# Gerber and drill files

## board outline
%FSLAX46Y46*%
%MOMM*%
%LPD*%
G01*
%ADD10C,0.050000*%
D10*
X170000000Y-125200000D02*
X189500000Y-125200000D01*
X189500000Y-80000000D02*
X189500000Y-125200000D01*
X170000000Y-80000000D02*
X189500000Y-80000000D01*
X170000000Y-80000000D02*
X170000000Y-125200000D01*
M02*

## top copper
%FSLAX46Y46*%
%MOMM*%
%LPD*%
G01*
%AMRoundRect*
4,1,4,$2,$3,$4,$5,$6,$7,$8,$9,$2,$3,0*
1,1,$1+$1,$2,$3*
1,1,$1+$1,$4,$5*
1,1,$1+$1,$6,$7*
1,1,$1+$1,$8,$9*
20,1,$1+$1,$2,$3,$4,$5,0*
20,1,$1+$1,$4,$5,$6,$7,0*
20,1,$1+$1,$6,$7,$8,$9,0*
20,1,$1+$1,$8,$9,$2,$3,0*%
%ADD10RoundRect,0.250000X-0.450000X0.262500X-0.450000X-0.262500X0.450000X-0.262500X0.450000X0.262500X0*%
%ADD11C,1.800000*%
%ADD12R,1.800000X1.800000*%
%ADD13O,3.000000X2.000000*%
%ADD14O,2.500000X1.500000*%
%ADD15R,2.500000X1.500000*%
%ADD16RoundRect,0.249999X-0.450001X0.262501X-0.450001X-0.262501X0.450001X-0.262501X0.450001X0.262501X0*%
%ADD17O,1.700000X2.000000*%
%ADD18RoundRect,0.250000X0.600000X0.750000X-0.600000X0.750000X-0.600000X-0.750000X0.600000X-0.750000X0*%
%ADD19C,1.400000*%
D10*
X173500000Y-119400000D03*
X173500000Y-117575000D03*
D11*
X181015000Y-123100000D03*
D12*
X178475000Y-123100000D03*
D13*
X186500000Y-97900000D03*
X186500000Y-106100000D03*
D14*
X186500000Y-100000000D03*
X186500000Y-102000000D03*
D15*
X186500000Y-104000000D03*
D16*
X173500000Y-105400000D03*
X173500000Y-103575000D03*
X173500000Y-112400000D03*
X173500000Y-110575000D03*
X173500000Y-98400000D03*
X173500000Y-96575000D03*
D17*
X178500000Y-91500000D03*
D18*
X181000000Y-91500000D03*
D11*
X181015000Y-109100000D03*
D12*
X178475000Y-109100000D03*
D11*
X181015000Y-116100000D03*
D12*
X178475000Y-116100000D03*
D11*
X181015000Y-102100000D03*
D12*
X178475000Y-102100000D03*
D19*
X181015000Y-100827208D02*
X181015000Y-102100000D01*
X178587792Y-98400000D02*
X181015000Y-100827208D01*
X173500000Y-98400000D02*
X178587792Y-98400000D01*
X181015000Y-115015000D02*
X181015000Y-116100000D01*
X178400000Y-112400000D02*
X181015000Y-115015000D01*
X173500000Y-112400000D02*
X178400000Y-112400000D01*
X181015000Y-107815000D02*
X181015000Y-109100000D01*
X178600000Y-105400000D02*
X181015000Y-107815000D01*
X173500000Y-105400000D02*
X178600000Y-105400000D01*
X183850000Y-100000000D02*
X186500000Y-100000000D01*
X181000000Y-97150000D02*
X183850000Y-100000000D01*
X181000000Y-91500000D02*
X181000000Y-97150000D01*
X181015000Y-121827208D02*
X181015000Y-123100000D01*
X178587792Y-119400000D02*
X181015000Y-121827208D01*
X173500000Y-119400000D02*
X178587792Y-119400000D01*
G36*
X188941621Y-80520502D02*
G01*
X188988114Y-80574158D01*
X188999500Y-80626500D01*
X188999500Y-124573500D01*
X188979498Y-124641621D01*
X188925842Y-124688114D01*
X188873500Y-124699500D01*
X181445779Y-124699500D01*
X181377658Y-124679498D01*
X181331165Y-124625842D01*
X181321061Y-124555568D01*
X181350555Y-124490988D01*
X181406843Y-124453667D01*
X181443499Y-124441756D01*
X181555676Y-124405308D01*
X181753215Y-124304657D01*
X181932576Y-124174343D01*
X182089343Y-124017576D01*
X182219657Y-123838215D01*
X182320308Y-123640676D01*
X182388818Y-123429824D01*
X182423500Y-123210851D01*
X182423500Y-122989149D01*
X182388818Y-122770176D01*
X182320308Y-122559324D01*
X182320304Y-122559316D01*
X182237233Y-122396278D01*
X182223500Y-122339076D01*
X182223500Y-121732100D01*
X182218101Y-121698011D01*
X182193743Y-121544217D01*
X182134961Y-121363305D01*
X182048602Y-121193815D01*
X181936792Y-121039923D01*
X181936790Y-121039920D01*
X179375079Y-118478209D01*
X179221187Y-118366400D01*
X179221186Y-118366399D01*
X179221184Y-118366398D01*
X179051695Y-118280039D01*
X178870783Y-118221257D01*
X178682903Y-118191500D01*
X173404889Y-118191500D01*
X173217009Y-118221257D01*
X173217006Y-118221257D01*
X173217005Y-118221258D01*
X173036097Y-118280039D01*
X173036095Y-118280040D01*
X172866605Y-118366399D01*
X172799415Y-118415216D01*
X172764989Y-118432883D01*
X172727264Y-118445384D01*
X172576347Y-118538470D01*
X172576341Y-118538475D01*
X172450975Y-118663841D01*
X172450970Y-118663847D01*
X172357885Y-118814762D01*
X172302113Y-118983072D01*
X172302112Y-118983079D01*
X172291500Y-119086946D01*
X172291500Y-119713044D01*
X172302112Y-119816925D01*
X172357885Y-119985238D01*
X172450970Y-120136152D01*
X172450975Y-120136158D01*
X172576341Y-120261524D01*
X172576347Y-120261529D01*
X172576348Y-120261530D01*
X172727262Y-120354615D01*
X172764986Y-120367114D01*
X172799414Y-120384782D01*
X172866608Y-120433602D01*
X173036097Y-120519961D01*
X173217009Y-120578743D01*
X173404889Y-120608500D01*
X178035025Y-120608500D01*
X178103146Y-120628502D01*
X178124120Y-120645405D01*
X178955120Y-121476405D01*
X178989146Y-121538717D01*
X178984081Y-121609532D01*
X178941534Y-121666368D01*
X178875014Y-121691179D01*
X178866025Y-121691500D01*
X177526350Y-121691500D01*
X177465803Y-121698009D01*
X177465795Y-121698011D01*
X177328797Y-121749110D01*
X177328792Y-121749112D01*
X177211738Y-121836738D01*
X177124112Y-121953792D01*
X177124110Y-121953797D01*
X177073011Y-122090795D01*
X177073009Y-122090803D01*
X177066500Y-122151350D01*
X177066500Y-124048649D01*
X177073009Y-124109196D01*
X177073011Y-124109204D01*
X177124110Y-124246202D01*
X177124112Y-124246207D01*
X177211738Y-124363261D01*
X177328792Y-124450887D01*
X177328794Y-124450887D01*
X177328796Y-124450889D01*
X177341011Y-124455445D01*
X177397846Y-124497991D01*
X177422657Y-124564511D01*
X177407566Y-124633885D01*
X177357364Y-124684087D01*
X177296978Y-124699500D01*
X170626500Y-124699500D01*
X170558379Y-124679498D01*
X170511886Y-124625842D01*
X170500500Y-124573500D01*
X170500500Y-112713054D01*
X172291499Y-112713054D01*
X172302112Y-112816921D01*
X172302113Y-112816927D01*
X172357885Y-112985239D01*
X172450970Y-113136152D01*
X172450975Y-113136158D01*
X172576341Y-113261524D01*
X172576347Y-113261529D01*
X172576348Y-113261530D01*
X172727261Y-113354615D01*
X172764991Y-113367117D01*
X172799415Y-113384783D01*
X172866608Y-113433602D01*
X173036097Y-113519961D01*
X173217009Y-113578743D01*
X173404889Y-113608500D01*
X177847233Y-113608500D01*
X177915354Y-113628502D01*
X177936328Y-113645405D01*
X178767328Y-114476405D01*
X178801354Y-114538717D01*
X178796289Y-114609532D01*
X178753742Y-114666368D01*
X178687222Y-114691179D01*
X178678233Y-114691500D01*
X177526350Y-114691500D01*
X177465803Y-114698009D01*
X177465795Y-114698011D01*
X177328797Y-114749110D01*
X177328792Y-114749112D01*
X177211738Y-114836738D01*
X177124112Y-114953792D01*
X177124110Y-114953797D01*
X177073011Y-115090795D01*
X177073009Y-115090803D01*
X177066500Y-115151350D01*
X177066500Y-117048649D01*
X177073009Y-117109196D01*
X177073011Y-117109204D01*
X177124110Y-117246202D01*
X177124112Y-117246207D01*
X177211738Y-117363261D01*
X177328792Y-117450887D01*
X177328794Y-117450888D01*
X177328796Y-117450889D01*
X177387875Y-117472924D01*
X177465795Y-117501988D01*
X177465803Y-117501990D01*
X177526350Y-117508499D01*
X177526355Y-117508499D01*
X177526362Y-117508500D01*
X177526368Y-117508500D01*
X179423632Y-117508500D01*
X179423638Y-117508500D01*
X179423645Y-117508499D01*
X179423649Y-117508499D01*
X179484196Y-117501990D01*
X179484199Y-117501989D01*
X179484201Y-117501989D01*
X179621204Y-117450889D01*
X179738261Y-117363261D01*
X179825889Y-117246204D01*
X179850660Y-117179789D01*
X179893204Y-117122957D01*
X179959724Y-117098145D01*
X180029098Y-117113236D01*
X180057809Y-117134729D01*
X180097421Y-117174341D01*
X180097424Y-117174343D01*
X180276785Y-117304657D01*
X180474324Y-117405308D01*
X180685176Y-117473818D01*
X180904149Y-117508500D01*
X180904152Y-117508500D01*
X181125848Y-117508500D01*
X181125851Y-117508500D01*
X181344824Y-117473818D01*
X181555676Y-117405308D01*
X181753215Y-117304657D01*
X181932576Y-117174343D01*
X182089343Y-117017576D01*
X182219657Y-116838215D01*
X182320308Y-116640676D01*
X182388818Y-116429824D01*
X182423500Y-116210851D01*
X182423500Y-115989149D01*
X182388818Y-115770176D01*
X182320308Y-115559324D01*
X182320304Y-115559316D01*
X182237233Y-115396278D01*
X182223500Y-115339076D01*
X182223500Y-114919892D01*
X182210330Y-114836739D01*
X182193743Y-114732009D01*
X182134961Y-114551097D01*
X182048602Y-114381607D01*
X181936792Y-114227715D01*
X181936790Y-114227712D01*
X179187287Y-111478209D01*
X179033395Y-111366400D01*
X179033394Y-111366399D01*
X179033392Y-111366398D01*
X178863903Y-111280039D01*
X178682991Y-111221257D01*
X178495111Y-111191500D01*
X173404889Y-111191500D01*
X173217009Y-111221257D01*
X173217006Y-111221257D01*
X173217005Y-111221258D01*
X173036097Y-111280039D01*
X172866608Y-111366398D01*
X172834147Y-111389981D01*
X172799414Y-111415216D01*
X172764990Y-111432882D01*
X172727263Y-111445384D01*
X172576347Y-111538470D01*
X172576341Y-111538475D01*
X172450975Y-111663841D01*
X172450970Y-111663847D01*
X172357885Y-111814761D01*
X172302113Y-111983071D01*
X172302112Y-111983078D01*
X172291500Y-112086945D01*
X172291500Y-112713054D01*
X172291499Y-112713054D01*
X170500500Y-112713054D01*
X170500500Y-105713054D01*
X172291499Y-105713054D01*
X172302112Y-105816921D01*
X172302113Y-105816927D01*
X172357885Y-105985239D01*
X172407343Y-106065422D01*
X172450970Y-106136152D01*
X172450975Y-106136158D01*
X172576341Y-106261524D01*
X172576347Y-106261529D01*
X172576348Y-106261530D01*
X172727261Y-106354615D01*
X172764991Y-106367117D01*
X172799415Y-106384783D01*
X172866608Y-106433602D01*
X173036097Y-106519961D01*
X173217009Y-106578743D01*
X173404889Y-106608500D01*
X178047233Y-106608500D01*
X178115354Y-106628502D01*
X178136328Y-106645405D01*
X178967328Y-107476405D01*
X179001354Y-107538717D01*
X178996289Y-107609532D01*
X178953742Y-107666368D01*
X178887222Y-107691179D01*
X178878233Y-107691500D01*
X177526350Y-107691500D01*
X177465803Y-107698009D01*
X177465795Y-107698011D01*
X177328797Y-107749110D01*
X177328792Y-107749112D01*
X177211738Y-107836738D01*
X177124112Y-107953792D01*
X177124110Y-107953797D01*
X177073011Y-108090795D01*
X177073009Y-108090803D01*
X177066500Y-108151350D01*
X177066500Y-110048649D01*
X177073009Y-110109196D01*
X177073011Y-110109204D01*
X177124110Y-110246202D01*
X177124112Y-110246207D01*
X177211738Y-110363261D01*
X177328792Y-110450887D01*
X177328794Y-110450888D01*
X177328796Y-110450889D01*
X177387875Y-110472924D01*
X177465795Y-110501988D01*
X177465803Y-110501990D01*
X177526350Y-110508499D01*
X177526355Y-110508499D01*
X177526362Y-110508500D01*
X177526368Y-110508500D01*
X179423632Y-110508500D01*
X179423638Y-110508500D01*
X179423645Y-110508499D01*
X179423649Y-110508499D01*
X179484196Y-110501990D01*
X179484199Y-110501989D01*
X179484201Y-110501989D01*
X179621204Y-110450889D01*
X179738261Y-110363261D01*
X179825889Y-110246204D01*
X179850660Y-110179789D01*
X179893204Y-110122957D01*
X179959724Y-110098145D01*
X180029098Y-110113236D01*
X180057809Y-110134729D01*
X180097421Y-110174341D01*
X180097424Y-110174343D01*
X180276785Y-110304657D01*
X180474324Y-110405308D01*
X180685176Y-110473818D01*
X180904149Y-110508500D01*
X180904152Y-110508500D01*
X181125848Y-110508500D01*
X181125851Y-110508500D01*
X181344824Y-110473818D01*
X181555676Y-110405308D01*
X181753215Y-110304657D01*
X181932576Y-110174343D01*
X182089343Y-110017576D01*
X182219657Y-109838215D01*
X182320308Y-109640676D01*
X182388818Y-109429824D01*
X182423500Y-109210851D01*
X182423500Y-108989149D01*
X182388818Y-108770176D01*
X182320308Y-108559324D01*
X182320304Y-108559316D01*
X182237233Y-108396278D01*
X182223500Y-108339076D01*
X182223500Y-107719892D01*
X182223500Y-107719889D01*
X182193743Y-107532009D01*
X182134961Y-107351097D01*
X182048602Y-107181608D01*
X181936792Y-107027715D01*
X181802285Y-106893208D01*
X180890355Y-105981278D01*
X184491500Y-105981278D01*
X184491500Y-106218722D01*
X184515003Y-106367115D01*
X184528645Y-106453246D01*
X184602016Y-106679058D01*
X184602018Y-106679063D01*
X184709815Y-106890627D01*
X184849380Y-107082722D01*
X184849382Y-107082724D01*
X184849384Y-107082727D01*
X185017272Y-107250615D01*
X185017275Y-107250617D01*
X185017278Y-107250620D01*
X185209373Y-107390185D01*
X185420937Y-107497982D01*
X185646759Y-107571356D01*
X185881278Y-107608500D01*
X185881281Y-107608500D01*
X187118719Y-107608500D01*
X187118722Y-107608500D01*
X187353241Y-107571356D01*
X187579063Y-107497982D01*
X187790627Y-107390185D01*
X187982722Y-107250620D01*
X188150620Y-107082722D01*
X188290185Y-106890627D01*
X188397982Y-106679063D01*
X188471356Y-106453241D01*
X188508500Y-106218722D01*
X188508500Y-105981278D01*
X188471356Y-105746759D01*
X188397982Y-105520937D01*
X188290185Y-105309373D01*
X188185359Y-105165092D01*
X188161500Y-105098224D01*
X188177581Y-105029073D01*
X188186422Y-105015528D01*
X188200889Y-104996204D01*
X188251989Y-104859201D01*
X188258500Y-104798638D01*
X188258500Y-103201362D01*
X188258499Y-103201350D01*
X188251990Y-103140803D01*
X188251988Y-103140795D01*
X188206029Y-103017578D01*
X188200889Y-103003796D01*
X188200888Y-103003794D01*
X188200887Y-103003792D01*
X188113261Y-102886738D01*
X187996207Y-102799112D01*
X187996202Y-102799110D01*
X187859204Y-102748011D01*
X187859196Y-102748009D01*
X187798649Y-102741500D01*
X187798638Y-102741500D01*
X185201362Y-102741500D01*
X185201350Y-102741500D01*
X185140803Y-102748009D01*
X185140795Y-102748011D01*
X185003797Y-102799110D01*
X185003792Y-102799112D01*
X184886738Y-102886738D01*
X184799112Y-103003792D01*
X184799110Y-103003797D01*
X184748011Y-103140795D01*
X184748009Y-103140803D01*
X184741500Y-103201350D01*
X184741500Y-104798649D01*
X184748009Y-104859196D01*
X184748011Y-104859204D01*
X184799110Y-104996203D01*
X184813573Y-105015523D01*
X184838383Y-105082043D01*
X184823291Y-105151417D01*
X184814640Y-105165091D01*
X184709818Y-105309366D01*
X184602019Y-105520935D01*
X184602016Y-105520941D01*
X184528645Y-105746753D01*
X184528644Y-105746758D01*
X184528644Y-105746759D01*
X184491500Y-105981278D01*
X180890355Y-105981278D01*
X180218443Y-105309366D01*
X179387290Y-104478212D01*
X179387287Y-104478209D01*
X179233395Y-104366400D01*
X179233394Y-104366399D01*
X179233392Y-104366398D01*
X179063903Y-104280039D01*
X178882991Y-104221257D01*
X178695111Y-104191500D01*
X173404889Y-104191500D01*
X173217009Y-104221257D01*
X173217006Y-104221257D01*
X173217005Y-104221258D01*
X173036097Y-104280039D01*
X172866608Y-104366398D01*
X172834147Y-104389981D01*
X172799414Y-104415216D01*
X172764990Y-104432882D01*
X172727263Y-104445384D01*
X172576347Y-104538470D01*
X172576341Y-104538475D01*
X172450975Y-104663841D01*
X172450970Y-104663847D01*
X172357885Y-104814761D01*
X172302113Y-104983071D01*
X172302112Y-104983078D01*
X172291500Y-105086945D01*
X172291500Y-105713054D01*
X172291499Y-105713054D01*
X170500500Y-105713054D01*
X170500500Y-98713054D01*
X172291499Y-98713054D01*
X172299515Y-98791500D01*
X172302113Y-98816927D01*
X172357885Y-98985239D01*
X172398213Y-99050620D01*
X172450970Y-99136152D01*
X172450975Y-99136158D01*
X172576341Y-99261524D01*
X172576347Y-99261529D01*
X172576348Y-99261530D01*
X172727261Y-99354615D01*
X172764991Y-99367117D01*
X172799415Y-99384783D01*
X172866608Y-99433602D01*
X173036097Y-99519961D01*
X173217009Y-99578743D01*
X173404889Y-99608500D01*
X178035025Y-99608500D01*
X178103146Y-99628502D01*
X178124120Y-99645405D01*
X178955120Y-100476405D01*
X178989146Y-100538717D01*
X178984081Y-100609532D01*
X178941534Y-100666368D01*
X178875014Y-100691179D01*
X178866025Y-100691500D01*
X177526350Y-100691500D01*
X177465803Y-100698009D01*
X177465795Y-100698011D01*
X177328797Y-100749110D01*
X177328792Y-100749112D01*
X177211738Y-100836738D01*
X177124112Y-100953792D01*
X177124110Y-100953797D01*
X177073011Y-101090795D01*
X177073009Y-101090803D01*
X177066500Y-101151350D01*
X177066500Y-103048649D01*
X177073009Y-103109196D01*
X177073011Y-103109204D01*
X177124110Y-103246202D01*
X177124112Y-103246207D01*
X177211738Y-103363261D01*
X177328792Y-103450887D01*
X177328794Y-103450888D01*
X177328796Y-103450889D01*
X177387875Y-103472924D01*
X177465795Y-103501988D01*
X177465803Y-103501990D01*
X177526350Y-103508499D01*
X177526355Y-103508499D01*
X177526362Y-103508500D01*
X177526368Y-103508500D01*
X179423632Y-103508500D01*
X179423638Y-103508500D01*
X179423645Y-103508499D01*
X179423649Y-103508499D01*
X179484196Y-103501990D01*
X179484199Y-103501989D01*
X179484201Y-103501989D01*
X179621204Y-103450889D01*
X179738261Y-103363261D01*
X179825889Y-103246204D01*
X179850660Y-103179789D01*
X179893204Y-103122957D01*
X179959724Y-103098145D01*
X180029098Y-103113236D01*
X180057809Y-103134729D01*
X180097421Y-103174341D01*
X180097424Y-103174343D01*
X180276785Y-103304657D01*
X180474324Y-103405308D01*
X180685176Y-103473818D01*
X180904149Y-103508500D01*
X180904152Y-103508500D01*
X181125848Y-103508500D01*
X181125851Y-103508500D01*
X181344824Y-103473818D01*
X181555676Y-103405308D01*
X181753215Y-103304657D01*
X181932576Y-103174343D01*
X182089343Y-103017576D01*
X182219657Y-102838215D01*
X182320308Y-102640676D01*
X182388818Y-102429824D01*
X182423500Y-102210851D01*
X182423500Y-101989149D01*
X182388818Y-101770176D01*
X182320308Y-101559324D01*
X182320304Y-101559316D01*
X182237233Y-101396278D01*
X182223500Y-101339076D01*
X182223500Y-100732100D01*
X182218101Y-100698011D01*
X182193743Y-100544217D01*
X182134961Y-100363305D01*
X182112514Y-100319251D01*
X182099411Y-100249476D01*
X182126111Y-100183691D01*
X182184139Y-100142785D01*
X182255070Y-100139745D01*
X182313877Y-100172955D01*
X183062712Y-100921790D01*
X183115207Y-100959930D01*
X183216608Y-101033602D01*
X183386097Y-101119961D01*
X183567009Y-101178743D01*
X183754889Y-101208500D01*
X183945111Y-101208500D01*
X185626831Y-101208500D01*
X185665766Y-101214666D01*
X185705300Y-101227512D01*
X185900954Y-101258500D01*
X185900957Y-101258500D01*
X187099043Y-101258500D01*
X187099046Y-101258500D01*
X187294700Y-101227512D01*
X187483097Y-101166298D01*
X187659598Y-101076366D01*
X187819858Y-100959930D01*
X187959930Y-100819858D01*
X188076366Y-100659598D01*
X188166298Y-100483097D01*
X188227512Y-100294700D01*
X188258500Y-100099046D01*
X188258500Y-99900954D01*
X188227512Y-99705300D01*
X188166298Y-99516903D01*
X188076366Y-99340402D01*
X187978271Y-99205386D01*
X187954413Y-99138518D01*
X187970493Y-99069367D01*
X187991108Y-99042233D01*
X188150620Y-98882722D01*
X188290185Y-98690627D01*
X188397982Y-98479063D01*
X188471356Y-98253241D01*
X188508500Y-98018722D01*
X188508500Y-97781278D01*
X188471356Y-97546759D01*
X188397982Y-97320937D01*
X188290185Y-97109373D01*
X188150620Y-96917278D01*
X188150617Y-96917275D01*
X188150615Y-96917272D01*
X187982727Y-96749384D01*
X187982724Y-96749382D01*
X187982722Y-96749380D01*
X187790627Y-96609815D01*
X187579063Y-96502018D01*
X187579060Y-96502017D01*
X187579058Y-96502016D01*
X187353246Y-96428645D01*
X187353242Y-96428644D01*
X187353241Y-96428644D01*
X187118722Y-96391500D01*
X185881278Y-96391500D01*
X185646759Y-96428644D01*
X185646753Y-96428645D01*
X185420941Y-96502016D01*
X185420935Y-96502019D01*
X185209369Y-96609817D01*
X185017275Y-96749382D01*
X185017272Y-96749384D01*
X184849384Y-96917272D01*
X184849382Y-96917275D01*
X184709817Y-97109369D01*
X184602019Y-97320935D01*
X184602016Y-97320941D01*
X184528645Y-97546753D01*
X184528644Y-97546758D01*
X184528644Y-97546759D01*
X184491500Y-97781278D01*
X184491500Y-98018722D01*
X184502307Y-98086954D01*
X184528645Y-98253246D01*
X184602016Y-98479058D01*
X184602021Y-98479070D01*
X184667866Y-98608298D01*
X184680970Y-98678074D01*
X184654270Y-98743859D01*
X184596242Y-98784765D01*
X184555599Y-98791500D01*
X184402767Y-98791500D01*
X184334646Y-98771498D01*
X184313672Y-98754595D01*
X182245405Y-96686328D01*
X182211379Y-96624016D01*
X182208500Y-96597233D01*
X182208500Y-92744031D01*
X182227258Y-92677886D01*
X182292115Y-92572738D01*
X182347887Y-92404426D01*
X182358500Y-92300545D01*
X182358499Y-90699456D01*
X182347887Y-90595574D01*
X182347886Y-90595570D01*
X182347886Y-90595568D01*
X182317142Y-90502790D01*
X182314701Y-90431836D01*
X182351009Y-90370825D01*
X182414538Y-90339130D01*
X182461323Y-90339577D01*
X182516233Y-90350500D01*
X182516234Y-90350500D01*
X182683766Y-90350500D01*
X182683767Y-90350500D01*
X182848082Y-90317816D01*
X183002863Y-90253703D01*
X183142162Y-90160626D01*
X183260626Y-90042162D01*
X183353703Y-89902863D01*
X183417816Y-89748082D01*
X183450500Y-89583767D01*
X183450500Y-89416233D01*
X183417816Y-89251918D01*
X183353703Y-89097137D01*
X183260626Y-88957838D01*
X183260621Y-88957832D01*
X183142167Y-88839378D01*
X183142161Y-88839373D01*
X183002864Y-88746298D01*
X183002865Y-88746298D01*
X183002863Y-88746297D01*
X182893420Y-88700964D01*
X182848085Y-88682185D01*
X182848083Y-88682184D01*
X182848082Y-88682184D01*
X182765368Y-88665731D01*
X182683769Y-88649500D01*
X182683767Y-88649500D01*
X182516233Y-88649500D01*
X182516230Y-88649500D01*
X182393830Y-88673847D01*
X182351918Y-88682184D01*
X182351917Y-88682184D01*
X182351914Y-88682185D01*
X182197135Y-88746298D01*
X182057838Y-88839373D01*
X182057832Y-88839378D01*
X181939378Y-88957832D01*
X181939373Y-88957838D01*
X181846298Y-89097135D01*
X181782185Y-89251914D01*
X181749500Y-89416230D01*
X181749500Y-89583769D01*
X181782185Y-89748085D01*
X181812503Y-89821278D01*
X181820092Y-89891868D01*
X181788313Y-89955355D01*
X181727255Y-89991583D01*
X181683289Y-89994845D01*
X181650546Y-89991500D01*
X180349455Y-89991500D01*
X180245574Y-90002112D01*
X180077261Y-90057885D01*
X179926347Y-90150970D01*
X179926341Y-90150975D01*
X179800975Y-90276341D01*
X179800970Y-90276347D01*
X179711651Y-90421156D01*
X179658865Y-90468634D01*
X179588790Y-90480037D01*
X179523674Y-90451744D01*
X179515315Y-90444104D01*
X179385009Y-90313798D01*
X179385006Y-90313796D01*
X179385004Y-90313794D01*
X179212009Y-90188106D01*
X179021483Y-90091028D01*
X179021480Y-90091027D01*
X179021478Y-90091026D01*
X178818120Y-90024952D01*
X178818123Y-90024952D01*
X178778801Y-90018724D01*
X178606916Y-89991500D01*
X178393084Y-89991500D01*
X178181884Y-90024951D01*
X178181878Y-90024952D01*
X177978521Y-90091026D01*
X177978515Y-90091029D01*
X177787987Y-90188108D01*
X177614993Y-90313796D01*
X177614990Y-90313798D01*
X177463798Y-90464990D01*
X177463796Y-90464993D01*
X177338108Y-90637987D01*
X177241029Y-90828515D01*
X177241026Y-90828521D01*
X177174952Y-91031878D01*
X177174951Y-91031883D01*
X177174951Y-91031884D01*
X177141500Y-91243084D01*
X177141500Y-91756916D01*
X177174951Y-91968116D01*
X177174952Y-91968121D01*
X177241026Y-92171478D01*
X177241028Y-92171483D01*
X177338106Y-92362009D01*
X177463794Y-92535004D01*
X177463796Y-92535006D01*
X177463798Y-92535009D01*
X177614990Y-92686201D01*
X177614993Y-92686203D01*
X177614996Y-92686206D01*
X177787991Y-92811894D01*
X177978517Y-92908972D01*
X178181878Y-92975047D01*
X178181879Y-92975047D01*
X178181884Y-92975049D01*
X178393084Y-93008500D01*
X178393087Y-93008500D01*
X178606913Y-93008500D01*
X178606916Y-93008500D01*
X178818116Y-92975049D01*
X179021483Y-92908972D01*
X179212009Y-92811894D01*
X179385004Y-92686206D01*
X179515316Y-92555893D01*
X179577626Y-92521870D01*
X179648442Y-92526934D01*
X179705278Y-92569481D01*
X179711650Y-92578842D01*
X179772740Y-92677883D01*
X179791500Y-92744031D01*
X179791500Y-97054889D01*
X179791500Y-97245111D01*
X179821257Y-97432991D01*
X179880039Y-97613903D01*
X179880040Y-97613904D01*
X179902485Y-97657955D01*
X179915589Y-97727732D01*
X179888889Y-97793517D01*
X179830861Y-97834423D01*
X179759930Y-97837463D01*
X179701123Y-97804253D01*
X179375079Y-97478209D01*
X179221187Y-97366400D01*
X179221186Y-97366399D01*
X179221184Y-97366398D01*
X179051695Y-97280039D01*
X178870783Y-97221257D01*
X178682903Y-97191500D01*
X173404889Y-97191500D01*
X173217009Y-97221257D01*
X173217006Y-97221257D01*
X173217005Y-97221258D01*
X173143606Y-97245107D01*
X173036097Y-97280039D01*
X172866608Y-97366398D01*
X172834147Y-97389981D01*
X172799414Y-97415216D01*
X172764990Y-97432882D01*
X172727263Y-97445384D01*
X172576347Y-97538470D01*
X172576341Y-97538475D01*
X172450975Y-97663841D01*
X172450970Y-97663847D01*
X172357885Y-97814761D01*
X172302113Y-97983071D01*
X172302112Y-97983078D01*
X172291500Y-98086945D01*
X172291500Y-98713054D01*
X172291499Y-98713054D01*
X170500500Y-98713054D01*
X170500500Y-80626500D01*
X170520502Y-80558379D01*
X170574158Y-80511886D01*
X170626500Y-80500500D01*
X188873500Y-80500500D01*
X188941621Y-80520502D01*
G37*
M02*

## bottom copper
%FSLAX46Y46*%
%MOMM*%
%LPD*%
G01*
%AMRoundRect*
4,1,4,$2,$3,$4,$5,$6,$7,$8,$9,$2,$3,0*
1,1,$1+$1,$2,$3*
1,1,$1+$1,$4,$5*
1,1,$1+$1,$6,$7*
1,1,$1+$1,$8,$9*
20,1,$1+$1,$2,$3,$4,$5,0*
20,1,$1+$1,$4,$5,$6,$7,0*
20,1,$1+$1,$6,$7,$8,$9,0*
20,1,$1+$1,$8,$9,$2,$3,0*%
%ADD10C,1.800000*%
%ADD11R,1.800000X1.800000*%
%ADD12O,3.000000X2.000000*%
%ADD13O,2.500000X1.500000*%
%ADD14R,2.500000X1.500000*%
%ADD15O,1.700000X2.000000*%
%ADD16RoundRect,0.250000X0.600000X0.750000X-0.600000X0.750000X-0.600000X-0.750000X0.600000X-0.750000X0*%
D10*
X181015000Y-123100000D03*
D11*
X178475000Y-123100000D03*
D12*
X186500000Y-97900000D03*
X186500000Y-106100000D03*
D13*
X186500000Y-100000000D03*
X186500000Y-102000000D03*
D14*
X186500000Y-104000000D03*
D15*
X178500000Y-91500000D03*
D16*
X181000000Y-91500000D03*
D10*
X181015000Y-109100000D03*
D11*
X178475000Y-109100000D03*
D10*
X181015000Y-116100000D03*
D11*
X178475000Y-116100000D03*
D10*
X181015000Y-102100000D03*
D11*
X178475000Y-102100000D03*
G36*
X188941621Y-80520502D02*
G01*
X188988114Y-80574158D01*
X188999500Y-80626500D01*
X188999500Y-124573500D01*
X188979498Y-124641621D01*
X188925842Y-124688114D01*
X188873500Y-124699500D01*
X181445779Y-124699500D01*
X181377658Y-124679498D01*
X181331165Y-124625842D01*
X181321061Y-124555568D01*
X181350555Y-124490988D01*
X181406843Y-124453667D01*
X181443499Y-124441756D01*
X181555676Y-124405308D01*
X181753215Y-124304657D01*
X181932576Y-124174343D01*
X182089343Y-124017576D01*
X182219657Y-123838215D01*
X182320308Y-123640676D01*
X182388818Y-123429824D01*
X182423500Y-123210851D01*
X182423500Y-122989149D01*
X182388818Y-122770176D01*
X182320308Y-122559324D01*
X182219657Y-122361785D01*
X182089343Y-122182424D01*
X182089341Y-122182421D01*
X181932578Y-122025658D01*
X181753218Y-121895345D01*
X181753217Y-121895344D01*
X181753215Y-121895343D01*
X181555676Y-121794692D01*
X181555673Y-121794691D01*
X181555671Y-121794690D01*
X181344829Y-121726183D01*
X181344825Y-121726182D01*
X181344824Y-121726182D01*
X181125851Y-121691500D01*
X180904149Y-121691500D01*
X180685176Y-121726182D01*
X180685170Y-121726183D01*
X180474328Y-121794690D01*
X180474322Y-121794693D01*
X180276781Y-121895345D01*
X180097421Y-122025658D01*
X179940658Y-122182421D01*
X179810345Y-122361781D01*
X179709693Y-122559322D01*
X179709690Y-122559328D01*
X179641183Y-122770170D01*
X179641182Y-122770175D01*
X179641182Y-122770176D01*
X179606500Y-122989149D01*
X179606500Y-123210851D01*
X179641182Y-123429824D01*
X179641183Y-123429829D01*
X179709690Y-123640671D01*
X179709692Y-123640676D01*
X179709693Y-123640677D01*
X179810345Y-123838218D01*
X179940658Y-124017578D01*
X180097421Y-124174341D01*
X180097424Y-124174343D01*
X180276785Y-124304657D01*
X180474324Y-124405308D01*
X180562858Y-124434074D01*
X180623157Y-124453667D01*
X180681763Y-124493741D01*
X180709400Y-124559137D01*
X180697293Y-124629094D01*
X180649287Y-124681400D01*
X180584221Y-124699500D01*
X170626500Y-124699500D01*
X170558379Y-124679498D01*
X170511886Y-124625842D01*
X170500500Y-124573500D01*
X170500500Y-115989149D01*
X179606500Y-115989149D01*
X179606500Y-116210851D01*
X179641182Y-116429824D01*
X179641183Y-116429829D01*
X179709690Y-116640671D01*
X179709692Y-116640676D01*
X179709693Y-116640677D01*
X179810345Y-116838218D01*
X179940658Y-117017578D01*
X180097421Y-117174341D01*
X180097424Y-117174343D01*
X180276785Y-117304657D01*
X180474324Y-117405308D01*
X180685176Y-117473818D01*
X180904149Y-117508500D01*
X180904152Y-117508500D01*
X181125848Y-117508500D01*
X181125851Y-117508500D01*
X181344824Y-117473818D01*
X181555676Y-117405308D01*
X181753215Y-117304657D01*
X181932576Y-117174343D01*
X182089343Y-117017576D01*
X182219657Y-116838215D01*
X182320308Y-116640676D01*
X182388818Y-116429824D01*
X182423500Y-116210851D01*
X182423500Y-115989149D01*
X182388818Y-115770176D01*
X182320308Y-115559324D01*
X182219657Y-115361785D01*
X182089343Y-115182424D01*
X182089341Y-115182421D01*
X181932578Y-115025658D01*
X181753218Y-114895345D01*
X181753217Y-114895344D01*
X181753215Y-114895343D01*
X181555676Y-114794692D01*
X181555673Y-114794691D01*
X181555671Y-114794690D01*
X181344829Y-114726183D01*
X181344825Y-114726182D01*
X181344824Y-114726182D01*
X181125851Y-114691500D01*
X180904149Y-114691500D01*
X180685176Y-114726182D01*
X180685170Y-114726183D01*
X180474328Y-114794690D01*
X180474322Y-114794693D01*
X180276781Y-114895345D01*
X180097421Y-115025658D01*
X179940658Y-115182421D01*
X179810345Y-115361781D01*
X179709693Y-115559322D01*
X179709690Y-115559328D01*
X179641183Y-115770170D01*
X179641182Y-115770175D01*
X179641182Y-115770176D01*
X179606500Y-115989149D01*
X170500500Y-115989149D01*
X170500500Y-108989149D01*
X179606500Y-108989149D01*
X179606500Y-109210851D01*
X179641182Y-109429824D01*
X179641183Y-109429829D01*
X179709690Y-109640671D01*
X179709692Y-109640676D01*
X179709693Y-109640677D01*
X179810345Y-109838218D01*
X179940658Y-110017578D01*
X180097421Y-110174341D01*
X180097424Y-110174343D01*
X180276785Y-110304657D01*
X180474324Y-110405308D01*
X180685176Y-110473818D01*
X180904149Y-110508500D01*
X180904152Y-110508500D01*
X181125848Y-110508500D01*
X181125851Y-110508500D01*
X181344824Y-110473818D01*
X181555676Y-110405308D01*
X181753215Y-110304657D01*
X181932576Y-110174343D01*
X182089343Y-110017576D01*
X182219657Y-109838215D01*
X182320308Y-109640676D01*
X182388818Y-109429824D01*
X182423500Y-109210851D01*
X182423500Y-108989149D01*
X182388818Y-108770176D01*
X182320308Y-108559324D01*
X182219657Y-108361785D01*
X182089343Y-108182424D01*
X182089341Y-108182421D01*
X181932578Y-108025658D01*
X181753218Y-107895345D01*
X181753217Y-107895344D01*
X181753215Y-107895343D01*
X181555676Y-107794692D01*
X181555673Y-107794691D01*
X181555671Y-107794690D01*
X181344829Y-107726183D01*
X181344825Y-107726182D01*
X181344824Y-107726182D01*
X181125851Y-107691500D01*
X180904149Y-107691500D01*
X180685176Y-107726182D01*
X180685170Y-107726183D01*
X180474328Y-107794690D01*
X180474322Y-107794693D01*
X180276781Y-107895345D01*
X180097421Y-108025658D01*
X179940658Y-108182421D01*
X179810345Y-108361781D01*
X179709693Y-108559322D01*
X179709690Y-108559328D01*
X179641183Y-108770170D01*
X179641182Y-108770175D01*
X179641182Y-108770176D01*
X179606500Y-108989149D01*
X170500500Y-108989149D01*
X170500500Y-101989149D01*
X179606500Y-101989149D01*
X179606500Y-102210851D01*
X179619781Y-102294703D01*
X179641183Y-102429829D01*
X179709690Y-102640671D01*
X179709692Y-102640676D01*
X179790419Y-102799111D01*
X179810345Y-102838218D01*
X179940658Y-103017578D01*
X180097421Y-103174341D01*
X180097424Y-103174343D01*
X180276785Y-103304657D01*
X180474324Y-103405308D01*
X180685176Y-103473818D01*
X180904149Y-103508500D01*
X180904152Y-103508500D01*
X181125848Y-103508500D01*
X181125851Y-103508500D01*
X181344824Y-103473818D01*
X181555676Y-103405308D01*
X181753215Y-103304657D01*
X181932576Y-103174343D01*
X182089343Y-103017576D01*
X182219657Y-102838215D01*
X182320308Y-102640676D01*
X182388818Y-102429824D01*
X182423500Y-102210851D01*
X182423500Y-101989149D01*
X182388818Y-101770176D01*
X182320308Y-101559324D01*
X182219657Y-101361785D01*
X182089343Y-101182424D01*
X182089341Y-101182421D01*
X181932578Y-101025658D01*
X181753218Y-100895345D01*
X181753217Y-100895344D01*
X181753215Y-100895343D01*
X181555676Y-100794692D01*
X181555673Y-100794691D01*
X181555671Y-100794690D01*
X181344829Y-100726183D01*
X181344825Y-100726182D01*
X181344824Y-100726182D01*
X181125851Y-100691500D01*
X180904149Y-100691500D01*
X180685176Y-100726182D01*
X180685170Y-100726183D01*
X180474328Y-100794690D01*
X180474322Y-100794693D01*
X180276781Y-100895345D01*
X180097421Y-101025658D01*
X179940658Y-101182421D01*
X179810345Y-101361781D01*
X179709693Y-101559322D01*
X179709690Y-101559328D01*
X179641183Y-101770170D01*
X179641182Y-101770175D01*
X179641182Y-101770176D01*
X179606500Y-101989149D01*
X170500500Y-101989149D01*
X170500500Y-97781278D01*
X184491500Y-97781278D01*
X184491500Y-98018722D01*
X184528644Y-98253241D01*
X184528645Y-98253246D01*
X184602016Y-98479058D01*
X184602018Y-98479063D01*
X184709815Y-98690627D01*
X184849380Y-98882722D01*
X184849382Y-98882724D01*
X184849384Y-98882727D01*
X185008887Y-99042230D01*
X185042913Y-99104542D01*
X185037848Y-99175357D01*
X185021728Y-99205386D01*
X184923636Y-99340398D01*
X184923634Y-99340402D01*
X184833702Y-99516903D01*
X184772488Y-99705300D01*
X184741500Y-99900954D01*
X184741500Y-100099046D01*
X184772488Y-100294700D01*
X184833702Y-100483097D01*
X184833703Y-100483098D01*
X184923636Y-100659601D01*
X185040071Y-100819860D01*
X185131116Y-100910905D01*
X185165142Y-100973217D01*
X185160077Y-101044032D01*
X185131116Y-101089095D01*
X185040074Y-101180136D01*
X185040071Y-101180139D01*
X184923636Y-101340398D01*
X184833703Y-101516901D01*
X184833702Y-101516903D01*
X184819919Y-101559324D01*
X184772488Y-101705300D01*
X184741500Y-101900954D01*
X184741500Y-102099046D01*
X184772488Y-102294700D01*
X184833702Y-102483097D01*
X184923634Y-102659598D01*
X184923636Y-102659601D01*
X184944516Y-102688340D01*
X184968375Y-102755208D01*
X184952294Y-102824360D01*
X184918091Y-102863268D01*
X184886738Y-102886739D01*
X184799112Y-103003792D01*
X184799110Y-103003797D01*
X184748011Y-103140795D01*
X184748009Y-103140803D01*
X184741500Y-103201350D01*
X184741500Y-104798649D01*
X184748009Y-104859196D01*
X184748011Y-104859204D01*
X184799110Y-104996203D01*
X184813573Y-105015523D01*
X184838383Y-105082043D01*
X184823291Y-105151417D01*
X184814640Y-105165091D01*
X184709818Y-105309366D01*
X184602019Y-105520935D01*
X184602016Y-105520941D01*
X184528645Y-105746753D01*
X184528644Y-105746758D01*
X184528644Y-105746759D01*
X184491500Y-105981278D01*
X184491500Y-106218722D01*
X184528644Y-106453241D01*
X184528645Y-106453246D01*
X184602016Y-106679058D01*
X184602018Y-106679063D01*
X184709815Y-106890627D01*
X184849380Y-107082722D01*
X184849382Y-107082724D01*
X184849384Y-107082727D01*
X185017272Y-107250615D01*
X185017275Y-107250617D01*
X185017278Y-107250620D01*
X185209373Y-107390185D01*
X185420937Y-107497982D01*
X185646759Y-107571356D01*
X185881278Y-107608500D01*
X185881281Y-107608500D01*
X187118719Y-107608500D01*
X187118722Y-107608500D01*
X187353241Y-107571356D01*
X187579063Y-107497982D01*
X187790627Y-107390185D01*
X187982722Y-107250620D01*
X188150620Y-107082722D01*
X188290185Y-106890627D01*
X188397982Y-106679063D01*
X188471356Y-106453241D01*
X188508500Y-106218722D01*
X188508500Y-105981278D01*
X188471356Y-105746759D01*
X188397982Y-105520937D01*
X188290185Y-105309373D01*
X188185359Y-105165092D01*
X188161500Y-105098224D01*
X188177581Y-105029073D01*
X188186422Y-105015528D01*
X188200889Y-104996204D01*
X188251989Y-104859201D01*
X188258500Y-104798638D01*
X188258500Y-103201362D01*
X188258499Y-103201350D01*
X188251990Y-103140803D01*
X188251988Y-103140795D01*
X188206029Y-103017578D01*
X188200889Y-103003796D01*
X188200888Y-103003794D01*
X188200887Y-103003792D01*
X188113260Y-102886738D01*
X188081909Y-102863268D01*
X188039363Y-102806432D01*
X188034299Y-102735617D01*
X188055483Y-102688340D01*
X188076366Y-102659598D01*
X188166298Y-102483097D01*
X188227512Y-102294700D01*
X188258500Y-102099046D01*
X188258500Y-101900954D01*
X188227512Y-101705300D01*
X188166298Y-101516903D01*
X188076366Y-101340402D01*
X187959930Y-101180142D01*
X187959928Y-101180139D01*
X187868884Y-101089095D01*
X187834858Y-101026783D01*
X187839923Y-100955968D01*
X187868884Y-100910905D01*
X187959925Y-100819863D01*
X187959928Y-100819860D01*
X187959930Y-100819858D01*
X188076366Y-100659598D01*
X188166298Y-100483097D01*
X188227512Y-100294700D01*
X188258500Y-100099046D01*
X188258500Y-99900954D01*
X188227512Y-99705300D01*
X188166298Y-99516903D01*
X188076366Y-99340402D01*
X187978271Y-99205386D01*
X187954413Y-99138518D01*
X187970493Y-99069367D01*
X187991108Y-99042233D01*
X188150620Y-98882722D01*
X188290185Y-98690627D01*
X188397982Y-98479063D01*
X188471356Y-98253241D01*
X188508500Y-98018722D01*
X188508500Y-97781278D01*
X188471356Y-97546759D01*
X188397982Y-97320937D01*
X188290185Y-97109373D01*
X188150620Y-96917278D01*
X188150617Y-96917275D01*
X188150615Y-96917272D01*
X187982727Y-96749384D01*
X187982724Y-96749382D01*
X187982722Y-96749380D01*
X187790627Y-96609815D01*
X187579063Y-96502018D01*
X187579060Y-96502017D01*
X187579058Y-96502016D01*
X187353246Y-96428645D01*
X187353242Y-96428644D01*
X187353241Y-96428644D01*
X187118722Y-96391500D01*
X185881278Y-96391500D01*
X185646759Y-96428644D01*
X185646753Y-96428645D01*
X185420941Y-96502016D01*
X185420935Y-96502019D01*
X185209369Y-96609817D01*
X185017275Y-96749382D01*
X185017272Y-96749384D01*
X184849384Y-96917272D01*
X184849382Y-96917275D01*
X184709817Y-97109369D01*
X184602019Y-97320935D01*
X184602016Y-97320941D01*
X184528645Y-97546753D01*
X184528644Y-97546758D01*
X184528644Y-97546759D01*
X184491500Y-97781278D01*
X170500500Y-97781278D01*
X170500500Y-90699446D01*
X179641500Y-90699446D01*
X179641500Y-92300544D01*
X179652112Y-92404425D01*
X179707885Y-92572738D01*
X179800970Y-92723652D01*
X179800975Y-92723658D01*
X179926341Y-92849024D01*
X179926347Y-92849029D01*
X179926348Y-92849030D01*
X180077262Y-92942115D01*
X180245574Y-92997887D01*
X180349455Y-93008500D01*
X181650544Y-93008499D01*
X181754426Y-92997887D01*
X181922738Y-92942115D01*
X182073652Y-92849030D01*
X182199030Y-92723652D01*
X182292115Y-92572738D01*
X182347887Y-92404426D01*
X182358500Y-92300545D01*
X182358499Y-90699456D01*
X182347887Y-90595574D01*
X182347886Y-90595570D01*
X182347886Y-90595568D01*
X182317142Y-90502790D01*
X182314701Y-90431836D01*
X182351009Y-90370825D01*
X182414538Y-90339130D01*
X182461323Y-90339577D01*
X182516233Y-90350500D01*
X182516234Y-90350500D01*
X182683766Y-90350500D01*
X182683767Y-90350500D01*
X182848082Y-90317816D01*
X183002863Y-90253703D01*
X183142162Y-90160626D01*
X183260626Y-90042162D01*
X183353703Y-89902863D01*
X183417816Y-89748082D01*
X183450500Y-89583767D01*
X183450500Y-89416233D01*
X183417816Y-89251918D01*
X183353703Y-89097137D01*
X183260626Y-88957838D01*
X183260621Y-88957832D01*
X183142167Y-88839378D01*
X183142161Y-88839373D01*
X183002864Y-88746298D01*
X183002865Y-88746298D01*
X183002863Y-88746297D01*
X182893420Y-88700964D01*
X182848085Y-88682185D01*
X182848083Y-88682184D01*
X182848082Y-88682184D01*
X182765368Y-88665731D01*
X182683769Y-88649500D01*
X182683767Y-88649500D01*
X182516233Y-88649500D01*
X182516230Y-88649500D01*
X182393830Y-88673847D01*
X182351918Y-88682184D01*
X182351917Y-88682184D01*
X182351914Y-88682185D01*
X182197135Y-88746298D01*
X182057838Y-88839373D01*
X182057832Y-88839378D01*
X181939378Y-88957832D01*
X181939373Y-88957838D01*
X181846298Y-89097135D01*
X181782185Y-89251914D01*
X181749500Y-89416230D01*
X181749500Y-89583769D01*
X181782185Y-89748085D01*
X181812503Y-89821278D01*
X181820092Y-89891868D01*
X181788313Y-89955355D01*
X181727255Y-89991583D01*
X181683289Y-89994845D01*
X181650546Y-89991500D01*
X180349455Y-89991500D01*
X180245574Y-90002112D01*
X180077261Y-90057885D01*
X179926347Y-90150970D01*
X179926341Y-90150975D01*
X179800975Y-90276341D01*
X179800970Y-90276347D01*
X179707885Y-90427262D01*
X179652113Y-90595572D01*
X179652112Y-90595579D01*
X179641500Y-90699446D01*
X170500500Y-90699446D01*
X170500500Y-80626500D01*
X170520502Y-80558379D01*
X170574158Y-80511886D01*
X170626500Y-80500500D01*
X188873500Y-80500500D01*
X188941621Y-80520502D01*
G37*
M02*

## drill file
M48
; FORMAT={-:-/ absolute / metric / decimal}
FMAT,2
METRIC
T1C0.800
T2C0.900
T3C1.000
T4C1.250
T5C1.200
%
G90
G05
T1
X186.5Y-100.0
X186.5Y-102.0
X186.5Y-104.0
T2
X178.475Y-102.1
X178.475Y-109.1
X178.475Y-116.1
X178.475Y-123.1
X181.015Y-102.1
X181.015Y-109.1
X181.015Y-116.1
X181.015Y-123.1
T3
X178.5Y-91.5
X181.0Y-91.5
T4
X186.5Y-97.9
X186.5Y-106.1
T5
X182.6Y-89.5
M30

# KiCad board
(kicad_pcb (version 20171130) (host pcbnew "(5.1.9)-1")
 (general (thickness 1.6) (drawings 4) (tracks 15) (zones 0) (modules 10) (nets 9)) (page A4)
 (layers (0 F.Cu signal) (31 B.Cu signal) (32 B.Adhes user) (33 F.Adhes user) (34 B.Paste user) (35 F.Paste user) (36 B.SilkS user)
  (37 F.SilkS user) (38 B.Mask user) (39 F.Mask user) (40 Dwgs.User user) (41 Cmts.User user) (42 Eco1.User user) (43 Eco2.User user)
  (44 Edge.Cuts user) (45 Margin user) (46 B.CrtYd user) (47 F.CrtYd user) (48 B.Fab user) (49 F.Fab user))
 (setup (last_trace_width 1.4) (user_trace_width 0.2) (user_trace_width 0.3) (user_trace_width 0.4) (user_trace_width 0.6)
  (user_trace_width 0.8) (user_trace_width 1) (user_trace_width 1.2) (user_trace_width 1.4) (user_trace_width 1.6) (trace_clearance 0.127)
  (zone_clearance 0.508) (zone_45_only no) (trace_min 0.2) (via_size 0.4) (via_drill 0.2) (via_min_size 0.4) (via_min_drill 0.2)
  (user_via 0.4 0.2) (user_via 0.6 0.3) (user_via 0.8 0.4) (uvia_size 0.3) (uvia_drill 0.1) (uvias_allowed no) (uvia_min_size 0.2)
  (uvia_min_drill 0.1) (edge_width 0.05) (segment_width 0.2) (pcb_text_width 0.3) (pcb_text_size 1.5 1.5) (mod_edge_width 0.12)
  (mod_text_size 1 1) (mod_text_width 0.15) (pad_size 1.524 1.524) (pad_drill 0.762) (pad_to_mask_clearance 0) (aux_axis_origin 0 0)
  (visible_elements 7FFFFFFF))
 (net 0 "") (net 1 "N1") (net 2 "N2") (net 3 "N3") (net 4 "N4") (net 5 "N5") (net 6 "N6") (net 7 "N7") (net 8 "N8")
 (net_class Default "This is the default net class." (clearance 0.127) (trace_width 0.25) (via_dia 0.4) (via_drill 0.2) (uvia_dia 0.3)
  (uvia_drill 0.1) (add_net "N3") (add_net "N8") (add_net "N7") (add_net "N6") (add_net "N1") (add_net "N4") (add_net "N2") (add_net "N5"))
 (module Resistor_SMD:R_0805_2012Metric (layer F.Cu) (at 173.5 118.4875 270)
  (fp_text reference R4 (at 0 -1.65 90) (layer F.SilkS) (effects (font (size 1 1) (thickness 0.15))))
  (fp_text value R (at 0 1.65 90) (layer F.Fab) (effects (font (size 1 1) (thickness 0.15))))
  (pad 2 smd roundrect (at 0.9125 0 270) (size 1.025 1.4) (layers F.Cu F.Paste F.Mask) (roundrect_rratio 0.243902) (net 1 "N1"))
  (pad 1 smd roundrect (at -0.9125 0 270) (size 1.025 1.4) (layers F.Cu F.Paste F.Mask) (roundrect_rratio 0.243902) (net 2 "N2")))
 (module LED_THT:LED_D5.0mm (layer B.Cu) (at 178.475 123.1)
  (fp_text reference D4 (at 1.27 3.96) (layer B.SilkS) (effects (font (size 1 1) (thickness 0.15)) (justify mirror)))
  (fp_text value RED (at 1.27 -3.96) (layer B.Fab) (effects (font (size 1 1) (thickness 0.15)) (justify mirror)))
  (pad 2 thru_hole circle (at 2.54 0) (size 1.8 1.8) (drill 0.9) (layers *.Cu *.Mask) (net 1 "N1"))
  (pad 1 thru_hole rect (at 0 0) (size 1.8 1.8) (drill 0.9) (layers *.Cu *.Mask) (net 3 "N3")))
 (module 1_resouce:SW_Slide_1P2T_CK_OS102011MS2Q (layer F.Cu) (at 186.5 104 90)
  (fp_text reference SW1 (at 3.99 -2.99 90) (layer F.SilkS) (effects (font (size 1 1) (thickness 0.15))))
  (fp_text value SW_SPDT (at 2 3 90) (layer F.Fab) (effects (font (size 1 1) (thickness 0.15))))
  (pad "" thru_hole oval (at 6.1 0 90) (size 2 3) (drill 1.25) (layers *.Cu *.Mask))
  (pad "" thru_hole oval (at -2.1 0 90) (size 2 3) (drill 1.25) (layers *.Cu *.Mask))
  (pad 3 thru_hole oval (at 4 0 90) (size 1.5 2.5) (drill 0.8) (layers *.Cu *.Mask) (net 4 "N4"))
  (pad 2 thru_hole oval (at 2 0 90) (size 1.5 2.5) (drill 0.8) (layers *.Cu *.Mask) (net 2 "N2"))
  (pad 1 thru_hole rect (at 0 0 90) (size 1.5 2.5) (drill 0.8) (layers *.Cu *.Mask) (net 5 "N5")))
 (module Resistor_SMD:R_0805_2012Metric (layer F.Cu) (at 173.5 104.4875 270)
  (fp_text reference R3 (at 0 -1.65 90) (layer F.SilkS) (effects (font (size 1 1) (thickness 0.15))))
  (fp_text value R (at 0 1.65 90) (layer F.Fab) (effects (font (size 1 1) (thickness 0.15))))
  (pad 2 smd roundrect (at 0.9125 0 270) (size 1.025 1.4) (layers F.Cu F.Paste F.Mask) (roundrect_rratio 0.2439014634146341) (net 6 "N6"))
  (pad 1 smd roundrect (at -0.9125 0 270) (size 1.025 1.4) (layers F.Cu F.Paste F.Mask) (roundrect_rratio 0.2439014634146341) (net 2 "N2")))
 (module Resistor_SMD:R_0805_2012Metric (layer F.Cu) (at 173.5 111.4875 270)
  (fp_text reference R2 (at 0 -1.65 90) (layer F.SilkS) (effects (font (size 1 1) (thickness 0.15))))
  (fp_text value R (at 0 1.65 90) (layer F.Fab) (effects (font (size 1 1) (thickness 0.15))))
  (pad 2 smd roundrect (at 0.9125 0 270) (size 1.025 1.4) (layers F.Cu F.Paste F.Mask) (roundrect_rratio 0.2439014634146341) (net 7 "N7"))
  (pad 1 smd roundrect (at -0.9125 0 270) (size 1.025 1.4) (layers F.Cu F.Paste F.Mask) (roundrect_rratio 0.2439014634146341) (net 2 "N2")))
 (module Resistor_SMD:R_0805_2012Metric (layer F.Cu) (at 173.5 97.4875 270)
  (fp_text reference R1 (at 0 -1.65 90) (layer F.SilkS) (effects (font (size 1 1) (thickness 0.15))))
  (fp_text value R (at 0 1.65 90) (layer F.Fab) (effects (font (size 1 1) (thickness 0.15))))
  (pad 2 smd roundrect (at 0.9125 0 270) (size 1.025 1.4) (layers F.Cu F.Paste F.Mask) (roundrect_rratio 0.2439014634146341) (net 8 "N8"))
  (pad 1 smd roundrect (at -0.9125 0 270) (size 1.025 1.4) (layers F.Cu F.Paste F.Mask) (roundrect_rratio 0.2439014634146341) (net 2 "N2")))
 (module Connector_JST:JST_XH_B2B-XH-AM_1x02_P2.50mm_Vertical (layer F.Cu) (at 181 91.5 180)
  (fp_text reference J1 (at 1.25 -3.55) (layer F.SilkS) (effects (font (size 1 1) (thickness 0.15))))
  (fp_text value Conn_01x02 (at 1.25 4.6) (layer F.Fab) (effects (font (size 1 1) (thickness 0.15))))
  (pad "" np_thru_hole circle (at -1.6 2 180) (size 1.2 1.2) (drill 1.2) (layers *.Cu *.Mask))
  (pad 2 thru_hole oval (at 2.5 0 180) (size 1.7 2) (drill 1) (layers *.Cu *.Mask) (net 3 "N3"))
  (pad 1 thru_hole roundrect (at 0 0 180) (size 1.7 2) (drill 1) (layers *.Cu *.Mask) (roundrect_rratio 0.1470588235294118) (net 4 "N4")))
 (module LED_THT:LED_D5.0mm (layer B.Cu) (at 178.475 109.1)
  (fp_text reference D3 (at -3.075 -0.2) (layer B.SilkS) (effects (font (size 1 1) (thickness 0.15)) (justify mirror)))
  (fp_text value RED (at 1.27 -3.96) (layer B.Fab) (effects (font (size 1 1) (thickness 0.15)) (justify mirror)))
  (pad 2 thru_hole circle (at 2.54 0) (size 1.8 1.8) (drill 0.9) (layers *.Cu *.Mask) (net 6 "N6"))
  (pad 1 thru_hole rect (at 0 0) (size 1.8 1.8) (drill 0.9) (layers *.Cu *.Mask) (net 3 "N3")))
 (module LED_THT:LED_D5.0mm (layer B.Cu) (at 178.475 116.1)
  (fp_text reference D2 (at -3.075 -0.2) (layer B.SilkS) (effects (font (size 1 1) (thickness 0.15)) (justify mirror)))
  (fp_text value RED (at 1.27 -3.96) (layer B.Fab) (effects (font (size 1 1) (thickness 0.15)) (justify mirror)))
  (pad 2 thru_hole circle (at 2.54 0) (size 1.8 1.8) (drill 0.9) (layers *.Cu *.Mask) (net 7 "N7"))
  (pad 1 thru_hole rect (at 0 0) (size 1.8 1.8) (drill 0.9) (layers *.Cu *.Mask) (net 3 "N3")))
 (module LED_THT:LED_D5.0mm (layer B.Cu) (at 178.475 102.1)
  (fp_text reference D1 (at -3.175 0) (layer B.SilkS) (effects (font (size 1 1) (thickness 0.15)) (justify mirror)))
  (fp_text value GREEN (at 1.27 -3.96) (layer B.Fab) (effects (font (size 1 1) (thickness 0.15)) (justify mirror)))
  (pad 2 thru_hole circle (at 2.54 0) (size 1.8 1.8) (drill 0.9) (layers *.Cu *.Mask) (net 8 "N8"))
  (pad 1 thru_hole rect (at 0 0) (size 1.8 1.8) (drill 0.9) (layers *.Cu *.Mask) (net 3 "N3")))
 (gr_line (start 170 125.2) (end 189.5 125.2) (layer Edge.Cuts) (width 0.05))
 (gr_line (start 189.5 80) (end 189.5 125.2) (layer Edge.Cuts) (width 0.05))
 (gr_line (start 170 80) (end 189.5 80) (layer Edge.Cuts) (width 0.05))
 (gr_line (start 170 80) (end 170 125.2) (layer Edge.Cuts) (width 0.05))
 (segment (start 181.015 100.827208) (end 181.015 102.1) (width 1.4) (layer F.Cu) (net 8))
 (segment (start 178.587792 98.4) (end 181.015 100.827208) (width 1.4) (layer F.Cu) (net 8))
 (segment (start 173.5 98.4) (end 178.587792 98.4) (width 1.4) (layer F.Cu) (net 8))
 (segment (start 181.015 115.015) (end 181.015 116.1) (width 1.4) (layer F.Cu) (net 7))
 (segment (start 178.4 112.4) (end 181.015 115.015) (width 1.4) (layer F.Cu) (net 7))
 (segment (start 173.5 112.4) (end 178.4 112.4) (width 1.4) (layer F.Cu) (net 7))
 (segment (start 181.015 107.815) (end 181.015 109.1) (width 1.4) (layer F.Cu) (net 6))
 (segment (start 178.6 105.4) (end 181.015 107.815) (width 1.4) (layer F.Cu) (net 6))
 (segment (start 173.5 105.4) (end 178.6 105.4) (width 1.4) (layer F.Cu) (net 6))
 (segment (start 183.85 100) (end 186.5 100) (width 1.4) (layer F.Cu) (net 4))
 (segment (start 181 97.15) (end 183.85 100) (width 1.4) (layer F.Cu) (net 4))
 (segment (start 181 91.5) (end 181 97.15) (width 1.4) (layer F.Cu) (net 4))
 (segment (start 181.015 121.827208) (end 181.015 123.1) (width 1.4) (layer F.Cu) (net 1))
 (segment (start 178.587792 119.4) (end 181.015 121.827208) (width 1.4) (layer F.Cu) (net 1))
 (segment (start 173.5 119.4) (end 178.587792 119.4) (width 1.4) (layer F.Cu) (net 1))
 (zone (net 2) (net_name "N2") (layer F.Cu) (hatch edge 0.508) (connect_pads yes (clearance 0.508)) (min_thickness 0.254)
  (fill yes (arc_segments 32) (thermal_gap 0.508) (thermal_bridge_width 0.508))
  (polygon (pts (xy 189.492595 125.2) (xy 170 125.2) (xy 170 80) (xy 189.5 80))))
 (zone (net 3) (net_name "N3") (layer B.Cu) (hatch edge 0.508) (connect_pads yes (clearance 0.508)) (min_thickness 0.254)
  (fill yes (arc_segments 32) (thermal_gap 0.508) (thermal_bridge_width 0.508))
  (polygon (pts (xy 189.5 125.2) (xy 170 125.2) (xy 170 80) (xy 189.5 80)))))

